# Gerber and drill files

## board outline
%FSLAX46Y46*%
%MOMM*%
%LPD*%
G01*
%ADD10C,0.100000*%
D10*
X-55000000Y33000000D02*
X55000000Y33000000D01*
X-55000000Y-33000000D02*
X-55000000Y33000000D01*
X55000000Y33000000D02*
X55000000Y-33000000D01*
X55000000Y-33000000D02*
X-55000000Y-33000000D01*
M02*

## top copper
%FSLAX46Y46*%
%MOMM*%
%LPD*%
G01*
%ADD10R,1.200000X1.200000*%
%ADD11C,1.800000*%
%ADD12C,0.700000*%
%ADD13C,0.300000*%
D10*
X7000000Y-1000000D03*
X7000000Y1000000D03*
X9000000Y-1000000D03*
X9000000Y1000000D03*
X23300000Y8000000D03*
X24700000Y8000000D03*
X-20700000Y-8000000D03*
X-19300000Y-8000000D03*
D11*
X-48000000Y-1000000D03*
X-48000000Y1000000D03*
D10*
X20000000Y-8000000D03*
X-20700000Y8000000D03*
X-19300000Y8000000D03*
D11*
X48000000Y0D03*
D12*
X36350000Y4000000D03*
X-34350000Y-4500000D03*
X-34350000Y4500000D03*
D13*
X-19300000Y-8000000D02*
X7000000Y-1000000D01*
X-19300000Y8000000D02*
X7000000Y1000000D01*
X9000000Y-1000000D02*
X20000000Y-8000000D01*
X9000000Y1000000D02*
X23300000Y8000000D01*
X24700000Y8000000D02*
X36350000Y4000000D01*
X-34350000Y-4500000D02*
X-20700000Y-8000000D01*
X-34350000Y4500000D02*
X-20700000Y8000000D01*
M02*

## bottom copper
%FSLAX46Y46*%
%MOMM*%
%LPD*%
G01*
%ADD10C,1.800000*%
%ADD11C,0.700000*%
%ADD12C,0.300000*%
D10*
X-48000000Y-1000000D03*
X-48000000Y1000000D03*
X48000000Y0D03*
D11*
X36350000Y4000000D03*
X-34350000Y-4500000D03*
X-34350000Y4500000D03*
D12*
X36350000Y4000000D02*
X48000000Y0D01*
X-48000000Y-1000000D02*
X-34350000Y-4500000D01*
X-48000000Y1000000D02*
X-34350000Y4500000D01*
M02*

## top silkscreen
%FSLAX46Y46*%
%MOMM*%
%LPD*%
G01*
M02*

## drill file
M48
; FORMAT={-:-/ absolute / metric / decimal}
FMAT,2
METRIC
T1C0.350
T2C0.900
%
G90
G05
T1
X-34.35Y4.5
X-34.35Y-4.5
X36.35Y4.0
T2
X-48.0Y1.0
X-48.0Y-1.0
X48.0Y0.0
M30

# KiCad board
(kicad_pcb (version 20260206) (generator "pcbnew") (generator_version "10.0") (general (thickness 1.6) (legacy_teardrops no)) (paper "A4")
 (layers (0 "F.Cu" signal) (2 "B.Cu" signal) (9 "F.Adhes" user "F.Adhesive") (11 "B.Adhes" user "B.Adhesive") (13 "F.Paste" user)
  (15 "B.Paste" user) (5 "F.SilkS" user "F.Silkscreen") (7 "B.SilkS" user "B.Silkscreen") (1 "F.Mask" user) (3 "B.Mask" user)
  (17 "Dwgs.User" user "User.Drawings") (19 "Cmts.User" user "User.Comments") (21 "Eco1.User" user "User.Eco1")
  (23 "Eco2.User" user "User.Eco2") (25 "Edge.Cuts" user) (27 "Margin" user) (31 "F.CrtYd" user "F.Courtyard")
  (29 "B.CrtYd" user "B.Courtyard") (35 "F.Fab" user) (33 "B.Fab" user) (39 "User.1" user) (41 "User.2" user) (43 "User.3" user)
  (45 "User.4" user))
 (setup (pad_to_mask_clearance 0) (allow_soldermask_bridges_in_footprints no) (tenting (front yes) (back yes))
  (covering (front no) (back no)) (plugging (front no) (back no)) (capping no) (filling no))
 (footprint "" (layer "F.Cu") (at 8 0)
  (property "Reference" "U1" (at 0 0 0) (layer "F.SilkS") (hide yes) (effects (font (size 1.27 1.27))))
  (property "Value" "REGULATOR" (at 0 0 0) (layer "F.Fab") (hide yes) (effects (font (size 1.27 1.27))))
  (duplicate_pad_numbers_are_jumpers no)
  (pad "1" smd rect (at -1 1) (size 1.2 1.2) (layers "F.Cu" "F.Mask" "F.Paste") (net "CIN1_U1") (thermal_bridge_angle 45))
  (pad "2" smd rect (at -1 -1) (size 1.2 1.2) (layers "F.Cu" "F.Mask" "F.Paste") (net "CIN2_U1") (thermal_bridge_angle 45))
  (pad "3" smd rect (at 1 1) (size 1.2 1.2) (layers "F.Cu" "F.Mask" "F.Paste") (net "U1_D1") (thermal_bridge_angle 45))
  (pad "4" smd rect (at 1 -1) (size 1.2 1.2) (layers "F.Cu" "F.Mask" "F.Paste") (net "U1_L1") (thermal_bridge_angle 45)))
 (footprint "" (layer "F.Cu") (at 24 -8)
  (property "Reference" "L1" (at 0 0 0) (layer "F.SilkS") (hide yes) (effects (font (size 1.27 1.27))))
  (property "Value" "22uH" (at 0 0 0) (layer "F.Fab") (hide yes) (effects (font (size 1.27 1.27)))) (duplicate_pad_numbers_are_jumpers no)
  (pad "1" smd rect (at -0.7 0) (size 1.2 1.2) (layers "F.Cu" "F.Mask" "F.Paste") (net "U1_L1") (thermal_bridge_angle 45))
  (pad "2" smd rect (at 0.7 0) (size 1.2 1.2) (layers "F.Cu" "F.Mask" "F.Paste") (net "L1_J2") (thermal_bridge_angle 45)))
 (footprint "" (layer "F.Cu") (at -20 8)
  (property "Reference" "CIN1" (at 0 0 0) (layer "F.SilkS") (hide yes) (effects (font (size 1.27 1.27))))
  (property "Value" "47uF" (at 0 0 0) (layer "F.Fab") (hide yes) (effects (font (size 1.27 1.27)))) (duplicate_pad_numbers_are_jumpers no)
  (pad "1" smd rect (at -0.7 0) (size 1.2 1.2) (layers "F.Cu" "F.Mask" "F.Paste") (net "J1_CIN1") (thermal_bridge_angle 45))
  (pad "2" smd rect (at 0.7 0) (size 1.2 1.2) (layers "F.Cu" "F.Mask" "F.Paste") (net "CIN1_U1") (thermal_bridge_angle 45)))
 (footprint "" (layer "F.Cu") (at -48 0)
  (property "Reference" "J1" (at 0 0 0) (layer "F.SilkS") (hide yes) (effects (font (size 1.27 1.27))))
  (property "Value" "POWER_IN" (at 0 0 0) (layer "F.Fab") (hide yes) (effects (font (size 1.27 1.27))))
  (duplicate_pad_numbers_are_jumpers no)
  (pad "1" thru_hole circle (at 0 1) (size 1.8 1.8) (drill 0.9) (layers "*.Cu" "*.Mask") (remove_unused_layers no) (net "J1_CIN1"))
  (pad "2" thru_hole circle (at 0 -1) (size 1.8 1.8) (drill 0.9) (layers "*.Cu" "*.Mask") (remove_unused_layers no) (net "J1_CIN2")))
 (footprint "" (layer "F.Cu") (at 20 8)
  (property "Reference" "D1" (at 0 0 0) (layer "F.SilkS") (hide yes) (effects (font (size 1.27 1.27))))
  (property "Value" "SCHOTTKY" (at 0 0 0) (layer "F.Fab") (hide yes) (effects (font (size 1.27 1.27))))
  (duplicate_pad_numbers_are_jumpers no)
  (pad "1" smd rect (at 0 0) (size 1.2 1.2) (layers "F.Cu" "F.Mask" "F.Paste") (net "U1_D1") (thermal_bridge_angle 45)))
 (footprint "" (layer "F.Cu") (at -20 -8)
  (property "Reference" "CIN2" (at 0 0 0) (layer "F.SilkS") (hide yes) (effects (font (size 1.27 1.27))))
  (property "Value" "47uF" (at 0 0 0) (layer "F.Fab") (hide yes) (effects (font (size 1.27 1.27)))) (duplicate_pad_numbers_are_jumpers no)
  (pad "1" smd rect (at -0.7 0) (size 1.2 1.2) (layers "F.Cu" "F.Mask" "F.Paste") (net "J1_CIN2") (thermal_bridge_angle 45))
  (pad "2" smd rect (at 0.7 0) (size 1.2 1.2) (layers "F.Cu" "F.Mask" "F.Paste") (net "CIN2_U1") (thermal_bridge_angle 45)))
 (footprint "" (layer "F.Cu") (at 48 0)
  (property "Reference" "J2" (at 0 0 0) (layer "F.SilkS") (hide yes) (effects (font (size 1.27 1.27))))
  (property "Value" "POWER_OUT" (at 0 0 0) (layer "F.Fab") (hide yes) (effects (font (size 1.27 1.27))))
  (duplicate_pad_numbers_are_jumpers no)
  (pad "1" thru_hole circle (at 0 0) (size 1.8 1.8) (drill 0.9) (layers "*.Cu" "*.Mask") (remove_unused_layers no) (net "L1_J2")))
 (gr_line (start -55 -33) (end 55 -33) (stroke (width 0.1) (type default)) (layer "Edge.Cuts"))
 (gr_line (start -55 33) (end -55 -33) (stroke (width 0.1) (type default)) (layer "Edge.Cuts"))
 (gr_line (start 55 -33) (end 55 33) (stroke (width 0.1) (type default)) (layer "Edge.Cuts"))
 (gr_line (start 55 33) (end -55 33) (stroke (width 0.1) (type default)) (layer "Edge.Cuts"))
 (segment (start -19.3 8) (end 7 1) (width 0.3) (layer "F.Cu") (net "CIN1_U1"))
 (segment (start -19.3 -8) (end 7 -1) (width 0.3) (layer "F.Cu") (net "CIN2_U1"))
 (segment (start 9 1) (end 20 8) (width 0.3) (layer "F.Cu") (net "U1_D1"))
 (segment (start 9 -1) (end 23.3 -8) (width 0.3) (layer "F.Cu") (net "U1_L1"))
 (segment (start 24.7 -8) (end 36.35 -4) (width 0.3) (layer "F.Cu") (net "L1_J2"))
 (via (at 36.35 -4) (size 0.7) (drill 0.35) (layers "F.Cu" "B.Cu") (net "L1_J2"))
 (segment (start 36.35 -4) (end 48 0) (width 0.3) (layer "B.Cu") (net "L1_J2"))
 (segment (start -34.35 4.5) (end -20.7 8) (width 0.3) (layer "F.Cu") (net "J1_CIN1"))
 (via (at -34.35 4.5) (size 0.7) (drill 0.35) (layers "F.Cu" "B.Cu") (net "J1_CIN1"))
 (segment (start -48 1) (end -34.35 4.5) (width 0.3) (layer "B.Cu") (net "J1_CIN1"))
 (segment (start -34.35 -4.5) (end -20.7 -8) (width 0.3) (layer "F.Cu") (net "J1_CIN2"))
 (via (at -34.35 -4.5) (size 0.7) (drill 0.35) (layers "F.Cu" "B.Cu") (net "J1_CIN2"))
 (segment (start -48 -1) (end -34.35 -4.5) (width 0.3) (layer "B.Cu") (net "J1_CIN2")))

